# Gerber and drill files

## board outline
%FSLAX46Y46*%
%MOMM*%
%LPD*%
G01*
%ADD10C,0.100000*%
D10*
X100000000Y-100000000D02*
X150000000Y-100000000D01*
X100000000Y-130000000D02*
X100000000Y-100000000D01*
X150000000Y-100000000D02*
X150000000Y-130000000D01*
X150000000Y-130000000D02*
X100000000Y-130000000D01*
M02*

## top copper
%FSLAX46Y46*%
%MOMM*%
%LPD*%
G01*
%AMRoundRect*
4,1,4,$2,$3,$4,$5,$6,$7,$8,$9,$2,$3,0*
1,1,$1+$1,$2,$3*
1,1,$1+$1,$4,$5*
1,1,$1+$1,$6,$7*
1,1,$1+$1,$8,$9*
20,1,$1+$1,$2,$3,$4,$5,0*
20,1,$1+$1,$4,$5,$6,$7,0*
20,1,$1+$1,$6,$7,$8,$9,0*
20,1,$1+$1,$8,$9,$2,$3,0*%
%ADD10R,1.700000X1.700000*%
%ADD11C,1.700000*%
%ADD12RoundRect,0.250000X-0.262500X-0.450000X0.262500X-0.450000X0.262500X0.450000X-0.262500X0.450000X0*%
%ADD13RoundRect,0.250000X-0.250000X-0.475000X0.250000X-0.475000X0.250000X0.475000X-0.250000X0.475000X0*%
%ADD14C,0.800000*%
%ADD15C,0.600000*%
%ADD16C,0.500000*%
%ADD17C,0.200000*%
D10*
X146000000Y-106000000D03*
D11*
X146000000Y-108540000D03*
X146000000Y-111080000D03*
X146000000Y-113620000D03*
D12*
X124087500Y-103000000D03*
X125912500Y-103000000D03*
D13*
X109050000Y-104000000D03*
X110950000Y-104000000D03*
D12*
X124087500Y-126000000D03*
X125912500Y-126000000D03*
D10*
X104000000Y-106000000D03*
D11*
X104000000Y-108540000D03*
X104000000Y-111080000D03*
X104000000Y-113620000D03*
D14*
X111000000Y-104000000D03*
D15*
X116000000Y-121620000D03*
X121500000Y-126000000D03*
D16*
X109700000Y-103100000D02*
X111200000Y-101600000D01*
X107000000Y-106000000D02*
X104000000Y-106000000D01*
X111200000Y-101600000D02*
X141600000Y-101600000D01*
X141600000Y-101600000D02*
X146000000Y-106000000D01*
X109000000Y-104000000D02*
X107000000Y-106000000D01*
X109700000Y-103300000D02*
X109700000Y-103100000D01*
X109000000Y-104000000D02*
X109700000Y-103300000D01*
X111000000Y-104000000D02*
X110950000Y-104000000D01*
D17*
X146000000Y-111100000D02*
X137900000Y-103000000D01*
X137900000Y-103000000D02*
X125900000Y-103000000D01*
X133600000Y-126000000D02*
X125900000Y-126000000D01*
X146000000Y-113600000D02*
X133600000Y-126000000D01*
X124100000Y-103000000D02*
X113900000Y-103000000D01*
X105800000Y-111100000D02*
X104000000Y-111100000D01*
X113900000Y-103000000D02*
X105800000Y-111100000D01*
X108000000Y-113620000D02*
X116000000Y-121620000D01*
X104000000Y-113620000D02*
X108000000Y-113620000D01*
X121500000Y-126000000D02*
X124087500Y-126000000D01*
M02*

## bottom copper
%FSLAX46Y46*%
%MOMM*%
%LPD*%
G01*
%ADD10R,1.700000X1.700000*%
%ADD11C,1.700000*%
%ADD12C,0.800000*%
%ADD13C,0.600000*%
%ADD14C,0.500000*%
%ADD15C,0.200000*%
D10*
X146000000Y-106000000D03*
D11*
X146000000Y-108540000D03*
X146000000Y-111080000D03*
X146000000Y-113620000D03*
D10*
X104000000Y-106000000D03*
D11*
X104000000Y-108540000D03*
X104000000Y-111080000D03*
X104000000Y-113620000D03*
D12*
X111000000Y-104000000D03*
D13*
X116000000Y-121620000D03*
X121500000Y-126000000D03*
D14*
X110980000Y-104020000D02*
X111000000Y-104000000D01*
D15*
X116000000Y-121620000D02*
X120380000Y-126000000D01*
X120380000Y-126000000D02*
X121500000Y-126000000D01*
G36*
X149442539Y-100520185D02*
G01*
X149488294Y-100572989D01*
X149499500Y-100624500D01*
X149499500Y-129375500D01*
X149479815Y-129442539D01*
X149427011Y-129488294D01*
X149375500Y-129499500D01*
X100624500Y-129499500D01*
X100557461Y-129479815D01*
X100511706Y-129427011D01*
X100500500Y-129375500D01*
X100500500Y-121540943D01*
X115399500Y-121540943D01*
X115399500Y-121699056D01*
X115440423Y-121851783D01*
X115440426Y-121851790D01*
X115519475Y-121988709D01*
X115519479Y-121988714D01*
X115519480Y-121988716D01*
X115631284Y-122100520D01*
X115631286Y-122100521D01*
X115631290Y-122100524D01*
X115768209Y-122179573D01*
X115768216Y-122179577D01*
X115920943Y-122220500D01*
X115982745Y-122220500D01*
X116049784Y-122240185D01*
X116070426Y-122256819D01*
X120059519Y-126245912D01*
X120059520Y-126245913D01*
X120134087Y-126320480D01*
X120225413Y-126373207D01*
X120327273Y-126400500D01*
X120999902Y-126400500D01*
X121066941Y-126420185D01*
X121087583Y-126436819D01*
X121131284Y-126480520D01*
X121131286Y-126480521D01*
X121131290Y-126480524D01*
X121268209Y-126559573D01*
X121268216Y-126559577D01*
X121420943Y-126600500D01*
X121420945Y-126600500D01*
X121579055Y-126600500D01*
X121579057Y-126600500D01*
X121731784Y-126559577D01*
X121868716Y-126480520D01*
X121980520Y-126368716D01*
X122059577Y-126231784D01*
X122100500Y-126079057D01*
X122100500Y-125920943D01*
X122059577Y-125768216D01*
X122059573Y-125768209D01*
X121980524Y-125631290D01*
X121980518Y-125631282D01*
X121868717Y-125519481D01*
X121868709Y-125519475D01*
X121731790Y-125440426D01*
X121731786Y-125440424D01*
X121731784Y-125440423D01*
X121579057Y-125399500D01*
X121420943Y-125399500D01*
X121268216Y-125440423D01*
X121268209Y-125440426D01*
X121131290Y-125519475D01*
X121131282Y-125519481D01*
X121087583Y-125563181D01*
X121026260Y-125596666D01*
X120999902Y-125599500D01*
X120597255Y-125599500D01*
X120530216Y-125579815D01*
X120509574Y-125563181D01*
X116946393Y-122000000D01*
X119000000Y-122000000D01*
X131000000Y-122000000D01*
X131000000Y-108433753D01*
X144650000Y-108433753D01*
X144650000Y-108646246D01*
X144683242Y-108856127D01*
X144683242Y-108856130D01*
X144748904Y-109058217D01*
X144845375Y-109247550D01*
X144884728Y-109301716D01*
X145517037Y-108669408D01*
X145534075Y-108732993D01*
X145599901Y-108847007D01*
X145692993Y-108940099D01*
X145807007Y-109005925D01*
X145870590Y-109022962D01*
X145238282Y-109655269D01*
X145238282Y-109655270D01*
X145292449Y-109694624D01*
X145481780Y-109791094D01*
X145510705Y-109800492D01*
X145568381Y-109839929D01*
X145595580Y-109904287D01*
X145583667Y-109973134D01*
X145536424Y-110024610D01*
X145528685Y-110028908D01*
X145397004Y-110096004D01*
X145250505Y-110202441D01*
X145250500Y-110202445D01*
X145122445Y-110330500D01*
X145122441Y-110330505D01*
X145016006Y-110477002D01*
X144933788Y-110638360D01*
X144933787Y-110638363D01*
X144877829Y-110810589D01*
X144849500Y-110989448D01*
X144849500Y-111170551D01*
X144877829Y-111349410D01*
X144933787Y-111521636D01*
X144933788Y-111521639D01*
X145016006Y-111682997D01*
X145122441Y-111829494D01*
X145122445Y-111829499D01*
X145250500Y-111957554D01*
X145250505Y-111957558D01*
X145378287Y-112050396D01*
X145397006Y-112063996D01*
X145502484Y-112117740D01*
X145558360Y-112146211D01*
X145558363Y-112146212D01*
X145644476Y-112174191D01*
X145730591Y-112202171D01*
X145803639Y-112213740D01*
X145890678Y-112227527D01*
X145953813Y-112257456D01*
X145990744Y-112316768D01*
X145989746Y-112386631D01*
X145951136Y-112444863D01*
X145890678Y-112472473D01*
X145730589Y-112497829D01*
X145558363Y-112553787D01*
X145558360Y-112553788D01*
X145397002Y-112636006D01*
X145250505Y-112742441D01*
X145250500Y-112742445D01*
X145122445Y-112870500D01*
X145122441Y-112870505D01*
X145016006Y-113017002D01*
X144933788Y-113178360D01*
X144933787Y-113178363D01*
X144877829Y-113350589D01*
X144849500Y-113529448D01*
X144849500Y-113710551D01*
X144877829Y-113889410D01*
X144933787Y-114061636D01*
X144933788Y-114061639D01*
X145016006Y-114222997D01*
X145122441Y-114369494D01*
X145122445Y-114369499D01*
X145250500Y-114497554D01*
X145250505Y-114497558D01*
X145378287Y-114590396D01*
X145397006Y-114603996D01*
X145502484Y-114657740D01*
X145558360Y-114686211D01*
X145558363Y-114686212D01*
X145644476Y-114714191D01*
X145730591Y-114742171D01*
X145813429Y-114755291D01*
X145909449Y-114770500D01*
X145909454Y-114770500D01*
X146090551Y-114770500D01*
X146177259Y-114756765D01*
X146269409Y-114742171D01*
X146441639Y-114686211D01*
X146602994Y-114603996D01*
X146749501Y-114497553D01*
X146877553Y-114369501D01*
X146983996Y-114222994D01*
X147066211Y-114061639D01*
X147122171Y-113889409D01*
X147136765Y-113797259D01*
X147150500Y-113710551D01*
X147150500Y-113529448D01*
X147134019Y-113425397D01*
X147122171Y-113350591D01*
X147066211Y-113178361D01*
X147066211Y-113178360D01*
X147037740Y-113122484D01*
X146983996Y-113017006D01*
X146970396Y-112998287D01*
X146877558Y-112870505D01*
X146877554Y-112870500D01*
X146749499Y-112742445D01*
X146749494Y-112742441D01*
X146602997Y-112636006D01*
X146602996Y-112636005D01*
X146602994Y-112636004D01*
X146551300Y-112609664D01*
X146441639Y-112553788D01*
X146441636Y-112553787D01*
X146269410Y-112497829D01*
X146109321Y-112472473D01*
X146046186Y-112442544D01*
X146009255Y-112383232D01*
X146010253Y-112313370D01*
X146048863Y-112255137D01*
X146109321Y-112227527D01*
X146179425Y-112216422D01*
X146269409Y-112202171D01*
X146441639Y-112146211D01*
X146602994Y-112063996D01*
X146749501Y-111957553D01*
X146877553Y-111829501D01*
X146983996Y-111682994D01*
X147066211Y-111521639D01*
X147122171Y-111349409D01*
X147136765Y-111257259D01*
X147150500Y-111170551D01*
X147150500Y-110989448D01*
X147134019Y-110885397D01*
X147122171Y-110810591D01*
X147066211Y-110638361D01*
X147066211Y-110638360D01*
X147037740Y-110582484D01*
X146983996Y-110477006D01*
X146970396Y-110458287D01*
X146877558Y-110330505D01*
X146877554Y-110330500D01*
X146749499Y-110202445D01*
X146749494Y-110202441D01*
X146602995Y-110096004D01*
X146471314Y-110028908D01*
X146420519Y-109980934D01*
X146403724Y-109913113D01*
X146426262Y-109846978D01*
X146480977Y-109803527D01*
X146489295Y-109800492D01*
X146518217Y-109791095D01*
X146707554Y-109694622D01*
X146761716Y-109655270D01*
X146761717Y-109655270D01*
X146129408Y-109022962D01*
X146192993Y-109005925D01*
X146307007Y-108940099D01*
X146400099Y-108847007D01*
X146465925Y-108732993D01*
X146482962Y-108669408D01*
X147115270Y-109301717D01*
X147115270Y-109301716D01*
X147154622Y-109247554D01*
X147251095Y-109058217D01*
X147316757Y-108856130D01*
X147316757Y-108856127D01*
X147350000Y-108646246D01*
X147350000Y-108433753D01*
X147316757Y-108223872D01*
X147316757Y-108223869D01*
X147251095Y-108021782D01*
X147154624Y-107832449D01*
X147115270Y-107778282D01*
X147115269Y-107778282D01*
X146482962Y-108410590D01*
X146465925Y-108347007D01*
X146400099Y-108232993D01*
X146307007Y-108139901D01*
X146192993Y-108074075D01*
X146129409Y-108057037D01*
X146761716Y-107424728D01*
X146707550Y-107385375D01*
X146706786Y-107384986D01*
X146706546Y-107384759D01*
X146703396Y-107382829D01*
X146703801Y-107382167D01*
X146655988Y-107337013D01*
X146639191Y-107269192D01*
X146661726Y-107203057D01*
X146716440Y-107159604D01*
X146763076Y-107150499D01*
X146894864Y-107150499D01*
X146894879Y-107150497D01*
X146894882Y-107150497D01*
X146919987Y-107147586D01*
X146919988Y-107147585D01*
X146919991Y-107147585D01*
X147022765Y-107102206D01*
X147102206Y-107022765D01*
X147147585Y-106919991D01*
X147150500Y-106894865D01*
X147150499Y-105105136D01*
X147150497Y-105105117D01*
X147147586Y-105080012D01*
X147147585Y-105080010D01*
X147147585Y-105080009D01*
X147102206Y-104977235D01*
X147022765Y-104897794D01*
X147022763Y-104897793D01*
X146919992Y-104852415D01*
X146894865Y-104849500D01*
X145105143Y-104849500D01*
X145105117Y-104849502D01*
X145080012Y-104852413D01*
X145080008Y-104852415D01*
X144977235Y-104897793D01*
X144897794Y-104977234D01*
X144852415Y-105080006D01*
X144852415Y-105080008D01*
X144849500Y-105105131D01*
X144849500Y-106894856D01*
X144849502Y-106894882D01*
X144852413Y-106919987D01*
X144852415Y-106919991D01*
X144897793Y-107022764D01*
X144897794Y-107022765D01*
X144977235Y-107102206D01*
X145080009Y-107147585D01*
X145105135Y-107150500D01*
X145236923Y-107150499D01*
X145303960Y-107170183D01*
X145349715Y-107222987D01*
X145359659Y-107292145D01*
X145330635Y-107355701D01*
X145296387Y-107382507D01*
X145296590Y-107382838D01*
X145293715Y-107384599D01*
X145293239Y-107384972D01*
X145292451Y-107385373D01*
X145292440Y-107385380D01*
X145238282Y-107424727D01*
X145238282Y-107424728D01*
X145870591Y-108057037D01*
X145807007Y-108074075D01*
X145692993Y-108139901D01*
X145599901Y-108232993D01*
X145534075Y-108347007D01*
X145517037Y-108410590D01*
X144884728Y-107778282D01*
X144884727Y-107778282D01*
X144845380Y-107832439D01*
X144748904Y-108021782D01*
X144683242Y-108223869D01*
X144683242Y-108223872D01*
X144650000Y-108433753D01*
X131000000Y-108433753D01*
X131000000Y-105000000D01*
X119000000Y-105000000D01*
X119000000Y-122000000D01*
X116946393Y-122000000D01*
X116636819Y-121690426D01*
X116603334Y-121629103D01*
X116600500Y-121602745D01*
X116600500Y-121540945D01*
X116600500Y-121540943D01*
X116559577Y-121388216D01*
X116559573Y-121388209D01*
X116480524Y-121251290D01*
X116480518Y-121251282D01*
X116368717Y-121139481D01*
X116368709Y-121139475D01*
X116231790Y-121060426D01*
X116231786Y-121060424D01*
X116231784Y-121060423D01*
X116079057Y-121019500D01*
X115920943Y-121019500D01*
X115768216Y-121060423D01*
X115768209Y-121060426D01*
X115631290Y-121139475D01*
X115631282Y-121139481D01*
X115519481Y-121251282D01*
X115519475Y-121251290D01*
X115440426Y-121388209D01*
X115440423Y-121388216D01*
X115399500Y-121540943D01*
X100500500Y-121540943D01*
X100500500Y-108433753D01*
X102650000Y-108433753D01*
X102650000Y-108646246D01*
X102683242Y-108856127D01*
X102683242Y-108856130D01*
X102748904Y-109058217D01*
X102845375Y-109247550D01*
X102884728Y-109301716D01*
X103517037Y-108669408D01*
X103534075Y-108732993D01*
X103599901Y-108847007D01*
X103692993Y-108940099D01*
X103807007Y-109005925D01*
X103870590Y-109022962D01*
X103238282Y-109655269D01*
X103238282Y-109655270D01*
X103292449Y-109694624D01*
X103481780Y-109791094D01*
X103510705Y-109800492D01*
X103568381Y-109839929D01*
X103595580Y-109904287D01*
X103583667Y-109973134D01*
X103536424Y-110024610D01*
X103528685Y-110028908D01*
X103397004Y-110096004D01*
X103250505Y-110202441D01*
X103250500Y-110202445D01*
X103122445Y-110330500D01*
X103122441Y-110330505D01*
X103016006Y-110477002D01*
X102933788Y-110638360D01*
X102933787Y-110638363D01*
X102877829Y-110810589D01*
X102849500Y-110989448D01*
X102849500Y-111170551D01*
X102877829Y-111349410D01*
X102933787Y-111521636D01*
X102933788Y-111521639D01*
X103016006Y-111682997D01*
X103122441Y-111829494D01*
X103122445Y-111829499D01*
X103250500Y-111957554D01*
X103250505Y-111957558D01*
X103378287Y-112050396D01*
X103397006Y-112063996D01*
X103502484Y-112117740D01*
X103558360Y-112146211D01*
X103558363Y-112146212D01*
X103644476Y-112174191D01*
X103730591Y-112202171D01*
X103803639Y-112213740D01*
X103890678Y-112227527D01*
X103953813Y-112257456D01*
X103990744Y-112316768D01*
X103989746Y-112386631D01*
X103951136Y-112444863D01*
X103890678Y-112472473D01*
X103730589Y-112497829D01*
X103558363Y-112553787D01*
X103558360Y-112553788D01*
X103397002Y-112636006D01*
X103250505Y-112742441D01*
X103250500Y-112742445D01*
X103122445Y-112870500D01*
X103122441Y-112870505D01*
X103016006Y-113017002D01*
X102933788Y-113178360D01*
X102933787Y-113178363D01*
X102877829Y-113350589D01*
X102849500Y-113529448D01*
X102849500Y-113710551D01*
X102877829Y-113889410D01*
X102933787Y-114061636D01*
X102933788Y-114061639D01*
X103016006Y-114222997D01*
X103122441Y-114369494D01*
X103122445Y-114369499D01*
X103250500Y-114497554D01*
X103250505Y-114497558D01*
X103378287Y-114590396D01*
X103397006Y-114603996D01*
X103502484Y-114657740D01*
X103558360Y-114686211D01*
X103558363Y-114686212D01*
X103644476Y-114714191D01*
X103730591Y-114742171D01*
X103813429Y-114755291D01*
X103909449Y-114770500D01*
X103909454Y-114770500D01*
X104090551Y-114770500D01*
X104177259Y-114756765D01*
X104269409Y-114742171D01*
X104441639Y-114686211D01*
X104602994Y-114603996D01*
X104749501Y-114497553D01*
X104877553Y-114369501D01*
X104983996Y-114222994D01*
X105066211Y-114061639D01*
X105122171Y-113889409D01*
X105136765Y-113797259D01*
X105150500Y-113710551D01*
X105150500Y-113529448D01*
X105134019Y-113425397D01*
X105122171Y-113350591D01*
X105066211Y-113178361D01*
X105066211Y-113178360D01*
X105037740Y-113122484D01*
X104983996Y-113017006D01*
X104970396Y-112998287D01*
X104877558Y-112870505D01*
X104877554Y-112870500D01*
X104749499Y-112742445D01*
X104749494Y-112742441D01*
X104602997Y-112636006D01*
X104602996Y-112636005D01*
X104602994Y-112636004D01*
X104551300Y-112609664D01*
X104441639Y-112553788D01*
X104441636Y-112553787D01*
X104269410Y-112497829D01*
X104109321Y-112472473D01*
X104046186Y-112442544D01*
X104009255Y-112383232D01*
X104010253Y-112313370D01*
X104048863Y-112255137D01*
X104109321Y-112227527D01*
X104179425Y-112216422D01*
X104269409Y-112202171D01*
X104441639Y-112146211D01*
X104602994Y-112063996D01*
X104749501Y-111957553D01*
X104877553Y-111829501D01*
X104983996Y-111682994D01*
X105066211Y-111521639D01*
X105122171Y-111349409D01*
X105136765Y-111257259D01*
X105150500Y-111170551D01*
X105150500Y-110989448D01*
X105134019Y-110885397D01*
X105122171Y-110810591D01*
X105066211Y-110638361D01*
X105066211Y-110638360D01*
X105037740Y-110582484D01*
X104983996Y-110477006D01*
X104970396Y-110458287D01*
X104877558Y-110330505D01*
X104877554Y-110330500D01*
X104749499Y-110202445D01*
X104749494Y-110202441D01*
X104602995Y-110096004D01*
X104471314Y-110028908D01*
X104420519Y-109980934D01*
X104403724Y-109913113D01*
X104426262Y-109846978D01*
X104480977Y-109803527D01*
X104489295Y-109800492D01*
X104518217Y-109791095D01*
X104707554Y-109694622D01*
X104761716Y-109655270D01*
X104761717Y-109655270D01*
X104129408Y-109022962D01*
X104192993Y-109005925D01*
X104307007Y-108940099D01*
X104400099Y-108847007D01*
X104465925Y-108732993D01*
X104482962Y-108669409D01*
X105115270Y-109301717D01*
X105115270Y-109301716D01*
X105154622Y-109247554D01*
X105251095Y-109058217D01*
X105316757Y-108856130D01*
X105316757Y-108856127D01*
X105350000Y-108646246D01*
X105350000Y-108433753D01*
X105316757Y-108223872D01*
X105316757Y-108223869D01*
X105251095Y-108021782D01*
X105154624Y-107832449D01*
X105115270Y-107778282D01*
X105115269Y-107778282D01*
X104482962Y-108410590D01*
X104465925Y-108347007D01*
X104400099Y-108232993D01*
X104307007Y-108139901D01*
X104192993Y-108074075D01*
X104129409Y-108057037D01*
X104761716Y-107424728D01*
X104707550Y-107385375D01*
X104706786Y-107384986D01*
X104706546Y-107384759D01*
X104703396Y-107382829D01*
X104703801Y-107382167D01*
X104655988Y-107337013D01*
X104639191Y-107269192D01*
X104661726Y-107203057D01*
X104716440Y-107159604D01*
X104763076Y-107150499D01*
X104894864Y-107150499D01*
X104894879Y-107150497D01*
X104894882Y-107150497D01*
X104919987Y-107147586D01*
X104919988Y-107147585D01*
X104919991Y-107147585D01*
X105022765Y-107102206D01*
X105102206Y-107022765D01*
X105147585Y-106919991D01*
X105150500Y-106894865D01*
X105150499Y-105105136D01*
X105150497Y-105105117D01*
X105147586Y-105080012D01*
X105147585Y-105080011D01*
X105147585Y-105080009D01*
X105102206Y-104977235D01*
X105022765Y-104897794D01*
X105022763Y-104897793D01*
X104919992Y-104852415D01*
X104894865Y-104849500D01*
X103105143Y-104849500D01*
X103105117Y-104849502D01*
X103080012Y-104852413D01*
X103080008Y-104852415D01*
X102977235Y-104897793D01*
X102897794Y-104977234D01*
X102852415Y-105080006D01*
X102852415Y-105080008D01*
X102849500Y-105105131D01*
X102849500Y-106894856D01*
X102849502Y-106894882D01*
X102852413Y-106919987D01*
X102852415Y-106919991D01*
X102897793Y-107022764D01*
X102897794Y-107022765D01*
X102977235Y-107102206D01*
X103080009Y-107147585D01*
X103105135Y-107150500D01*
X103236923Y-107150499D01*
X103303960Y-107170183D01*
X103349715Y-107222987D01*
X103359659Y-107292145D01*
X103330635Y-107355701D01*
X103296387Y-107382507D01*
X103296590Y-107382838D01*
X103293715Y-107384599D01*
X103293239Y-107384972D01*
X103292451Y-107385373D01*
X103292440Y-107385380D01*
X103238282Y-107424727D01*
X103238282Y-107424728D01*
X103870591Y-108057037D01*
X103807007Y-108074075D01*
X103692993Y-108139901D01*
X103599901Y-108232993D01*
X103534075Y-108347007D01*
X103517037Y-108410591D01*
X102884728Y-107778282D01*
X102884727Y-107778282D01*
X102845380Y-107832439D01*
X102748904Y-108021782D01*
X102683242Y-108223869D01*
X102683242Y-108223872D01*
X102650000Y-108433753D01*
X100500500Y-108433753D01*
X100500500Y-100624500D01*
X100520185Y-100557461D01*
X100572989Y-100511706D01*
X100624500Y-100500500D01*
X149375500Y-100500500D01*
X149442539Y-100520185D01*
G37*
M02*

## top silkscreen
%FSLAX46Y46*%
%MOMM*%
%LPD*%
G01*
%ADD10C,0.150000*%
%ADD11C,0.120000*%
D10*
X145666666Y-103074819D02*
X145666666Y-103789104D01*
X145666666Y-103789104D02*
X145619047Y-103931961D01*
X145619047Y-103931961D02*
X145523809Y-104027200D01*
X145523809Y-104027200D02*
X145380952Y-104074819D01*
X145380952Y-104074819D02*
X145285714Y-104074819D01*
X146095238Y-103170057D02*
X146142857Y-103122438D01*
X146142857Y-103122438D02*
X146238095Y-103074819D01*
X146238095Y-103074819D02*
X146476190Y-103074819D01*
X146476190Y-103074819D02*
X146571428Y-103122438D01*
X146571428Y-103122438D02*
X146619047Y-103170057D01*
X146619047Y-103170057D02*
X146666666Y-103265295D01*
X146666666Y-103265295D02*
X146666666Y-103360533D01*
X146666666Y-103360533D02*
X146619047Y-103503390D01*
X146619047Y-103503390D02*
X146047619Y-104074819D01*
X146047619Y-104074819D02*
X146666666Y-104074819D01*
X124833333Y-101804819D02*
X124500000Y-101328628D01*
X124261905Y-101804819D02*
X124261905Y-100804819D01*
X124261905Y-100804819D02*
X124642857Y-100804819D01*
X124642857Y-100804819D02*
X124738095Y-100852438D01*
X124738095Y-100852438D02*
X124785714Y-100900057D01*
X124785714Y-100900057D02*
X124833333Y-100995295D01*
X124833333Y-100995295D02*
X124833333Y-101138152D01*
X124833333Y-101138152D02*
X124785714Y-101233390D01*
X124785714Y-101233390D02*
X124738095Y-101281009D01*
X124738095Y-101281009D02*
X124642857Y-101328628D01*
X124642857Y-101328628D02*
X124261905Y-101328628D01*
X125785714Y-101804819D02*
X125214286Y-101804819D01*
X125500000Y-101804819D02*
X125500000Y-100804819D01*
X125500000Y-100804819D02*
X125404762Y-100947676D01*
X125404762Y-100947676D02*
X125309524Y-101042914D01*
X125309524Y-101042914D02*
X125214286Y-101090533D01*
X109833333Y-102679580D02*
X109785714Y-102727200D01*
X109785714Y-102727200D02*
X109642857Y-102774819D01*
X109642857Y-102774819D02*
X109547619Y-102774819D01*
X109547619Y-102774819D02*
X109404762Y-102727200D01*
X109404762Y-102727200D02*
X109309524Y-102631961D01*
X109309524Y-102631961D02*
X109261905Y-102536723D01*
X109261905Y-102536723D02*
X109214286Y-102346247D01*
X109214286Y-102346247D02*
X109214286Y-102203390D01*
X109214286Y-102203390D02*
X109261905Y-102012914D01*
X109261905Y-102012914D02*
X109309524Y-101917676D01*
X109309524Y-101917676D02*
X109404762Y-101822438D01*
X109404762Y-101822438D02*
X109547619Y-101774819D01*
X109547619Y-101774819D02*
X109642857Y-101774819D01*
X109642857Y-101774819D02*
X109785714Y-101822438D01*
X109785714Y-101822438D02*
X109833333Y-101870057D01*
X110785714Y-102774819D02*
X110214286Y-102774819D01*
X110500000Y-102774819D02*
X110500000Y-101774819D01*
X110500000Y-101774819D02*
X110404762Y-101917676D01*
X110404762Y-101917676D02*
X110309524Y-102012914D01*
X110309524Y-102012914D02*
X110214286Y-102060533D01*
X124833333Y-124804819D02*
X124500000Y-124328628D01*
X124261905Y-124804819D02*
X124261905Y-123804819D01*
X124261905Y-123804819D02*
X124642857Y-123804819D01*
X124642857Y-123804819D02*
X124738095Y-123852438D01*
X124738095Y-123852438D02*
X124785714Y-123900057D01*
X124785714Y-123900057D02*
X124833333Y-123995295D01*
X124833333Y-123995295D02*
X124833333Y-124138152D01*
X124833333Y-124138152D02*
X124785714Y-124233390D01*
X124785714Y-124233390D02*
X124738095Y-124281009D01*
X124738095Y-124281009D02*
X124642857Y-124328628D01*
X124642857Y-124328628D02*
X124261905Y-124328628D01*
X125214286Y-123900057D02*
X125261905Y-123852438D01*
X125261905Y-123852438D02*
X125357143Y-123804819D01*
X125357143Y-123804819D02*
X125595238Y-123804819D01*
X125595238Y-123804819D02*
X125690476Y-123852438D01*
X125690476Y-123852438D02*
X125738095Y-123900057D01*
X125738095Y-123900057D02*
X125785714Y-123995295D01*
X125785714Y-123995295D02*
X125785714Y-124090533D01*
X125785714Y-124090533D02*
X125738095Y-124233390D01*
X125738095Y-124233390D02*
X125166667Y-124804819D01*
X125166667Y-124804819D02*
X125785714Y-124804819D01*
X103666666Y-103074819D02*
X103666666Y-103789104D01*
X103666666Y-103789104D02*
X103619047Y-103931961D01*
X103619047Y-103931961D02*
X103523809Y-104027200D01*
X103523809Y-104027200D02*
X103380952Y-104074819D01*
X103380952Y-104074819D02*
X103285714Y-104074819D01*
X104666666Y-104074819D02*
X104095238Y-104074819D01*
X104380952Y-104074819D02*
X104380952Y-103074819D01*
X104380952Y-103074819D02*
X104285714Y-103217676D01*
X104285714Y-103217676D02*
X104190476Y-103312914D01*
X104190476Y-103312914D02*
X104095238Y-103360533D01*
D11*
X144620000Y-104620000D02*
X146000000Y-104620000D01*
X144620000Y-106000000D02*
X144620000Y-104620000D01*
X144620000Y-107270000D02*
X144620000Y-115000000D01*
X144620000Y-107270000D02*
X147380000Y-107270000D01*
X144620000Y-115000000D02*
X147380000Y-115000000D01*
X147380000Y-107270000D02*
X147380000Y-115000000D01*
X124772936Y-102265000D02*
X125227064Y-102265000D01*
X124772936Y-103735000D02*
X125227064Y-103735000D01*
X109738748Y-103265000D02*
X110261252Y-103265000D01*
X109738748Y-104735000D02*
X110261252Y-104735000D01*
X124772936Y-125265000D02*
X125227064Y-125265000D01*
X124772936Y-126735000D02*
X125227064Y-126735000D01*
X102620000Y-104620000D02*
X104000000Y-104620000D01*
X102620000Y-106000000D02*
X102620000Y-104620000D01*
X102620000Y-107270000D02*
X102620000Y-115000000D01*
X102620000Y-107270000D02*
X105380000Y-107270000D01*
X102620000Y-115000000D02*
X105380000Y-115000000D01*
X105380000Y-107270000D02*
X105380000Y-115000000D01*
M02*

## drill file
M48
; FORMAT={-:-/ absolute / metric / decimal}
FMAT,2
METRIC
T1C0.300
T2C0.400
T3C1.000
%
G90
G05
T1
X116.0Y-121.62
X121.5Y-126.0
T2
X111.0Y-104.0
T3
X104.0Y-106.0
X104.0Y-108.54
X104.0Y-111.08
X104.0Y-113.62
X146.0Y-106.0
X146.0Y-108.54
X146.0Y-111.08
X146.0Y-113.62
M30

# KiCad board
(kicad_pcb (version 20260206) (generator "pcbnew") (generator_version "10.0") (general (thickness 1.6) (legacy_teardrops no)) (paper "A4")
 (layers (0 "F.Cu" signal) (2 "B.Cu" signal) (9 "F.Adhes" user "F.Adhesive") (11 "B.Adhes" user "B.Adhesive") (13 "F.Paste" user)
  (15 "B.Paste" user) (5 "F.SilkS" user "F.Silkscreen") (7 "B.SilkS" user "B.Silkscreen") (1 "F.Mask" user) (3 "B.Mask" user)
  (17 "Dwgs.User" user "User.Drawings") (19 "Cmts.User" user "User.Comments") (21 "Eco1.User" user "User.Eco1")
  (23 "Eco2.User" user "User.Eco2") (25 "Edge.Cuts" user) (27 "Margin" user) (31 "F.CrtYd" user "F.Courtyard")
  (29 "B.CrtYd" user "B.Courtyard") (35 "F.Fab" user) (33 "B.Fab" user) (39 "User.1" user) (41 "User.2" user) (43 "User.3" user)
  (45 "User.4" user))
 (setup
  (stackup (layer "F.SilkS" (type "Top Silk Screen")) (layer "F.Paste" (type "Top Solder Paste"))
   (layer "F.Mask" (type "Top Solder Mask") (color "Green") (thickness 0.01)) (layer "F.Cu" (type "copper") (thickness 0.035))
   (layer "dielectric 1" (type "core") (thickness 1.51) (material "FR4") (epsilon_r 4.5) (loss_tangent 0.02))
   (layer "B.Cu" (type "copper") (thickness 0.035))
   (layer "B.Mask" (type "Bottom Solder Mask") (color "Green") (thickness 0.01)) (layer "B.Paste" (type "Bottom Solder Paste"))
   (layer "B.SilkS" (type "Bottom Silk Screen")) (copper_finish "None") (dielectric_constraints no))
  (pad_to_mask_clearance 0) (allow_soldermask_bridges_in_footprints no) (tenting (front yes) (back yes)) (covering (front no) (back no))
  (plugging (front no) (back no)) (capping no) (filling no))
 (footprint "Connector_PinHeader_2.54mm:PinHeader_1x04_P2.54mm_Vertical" (layer "F.Cu") (at 146 106)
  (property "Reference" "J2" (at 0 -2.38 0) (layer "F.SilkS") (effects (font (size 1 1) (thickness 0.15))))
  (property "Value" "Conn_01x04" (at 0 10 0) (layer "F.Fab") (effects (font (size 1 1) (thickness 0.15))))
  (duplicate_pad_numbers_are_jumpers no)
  (fp_line (start -1.38 -1.38) (end 0 -1.38) (stroke (width 0.12) (type solid)) (layer "F.SilkS"))
  (fp_line (start -1.38 0) (end -1.38 -1.38) (stroke (width 0.12) (type solid)) (layer "F.SilkS"))
  (fp_line (start -1.38 1.27) (end -1.38 9) (stroke (width 0.12) (type solid)) (layer "F.SilkS"))
  (fp_line (start -1.38 1.27) (end 1.38 1.27) (stroke (width 0.12) (type solid)) (layer "F.SilkS"))
  (fp_line (start -1.38 9) (end 1.38 9) (stroke (width 0.12) (type solid)) (layer "F.SilkS"))
  (fp_line (start 1.38 1.27) (end 1.38 9) (stroke (width 0.12) (type solid)) (layer "F.SilkS"))
  (pad "1" thru_hole rect (at 0 0) (size 1.7 1.7) (drill 1) (layers "*.Cu" "*.Mask") (remove_unused_layers no) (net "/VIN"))
  (pad "2" thru_hole circle (at 0 2.54) (size 1.7 1.7) (drill 1) (layers "*.Cu" "*.Mask") (remove_unused_layers no) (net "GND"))
  (pad "3" thru_hole circle (at 0 5.08) (size 1.7 1.7) (drill 1) (layers "*.Cu" "*.Mask") (remove_unused_layers no) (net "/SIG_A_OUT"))
  (pad "4" thru_hole circle (at 0 7.62) (size 1.7 1.7) (drill 1) (layers "*.Cu" "*.Mask") (remove_unused_layers no) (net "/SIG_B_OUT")))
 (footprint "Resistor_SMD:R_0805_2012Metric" (layer "F.Cu") (at 125 103)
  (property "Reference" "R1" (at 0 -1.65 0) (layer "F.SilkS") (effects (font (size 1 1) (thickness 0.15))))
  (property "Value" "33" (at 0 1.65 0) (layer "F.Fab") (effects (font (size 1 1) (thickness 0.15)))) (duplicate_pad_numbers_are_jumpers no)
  (fp_line (start -0.227064 -0.735) (end 0.227064 -0.735) (stroke (width 0.12) (type solid)) (layer "F.SilkS"))
  (fp_line (start -0.227064 0.735) (end 0.227064 0.735) (stroke (width 0.12) (type solid)) (layer "F.SilkS"))
  (pad "1" smd roundrect (at -0.9125 0) (size 1.025 1.4) (layers "F.Cu" "F.Mask" "F.Paste") (roundrect_rratio 0.243902) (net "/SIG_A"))
  (pad "2" smd roundrect (at 0.9125 0) (size 1.025 1.4) (layers "F.Cu" "F.Mask" "F.Paste") (roundrect_rratio 0.243902) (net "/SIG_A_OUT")))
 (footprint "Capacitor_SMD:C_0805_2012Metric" (layer "F.Cu") (at 110 104)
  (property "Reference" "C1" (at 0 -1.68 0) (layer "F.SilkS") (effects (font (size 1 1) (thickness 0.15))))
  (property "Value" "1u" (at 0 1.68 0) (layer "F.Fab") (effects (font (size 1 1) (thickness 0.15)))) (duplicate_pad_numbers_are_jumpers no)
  (fp_line (start -0.261252 -0.735) (end 0.261252 -0.735) (stroke (width 0.12) (type solid)) (layer "F.SilkS"))
  (fp_line (start -0.261252 0.735) (end 0.261252 0.735) (stroke (width 0.12) (type solid)) (layer "F.SilkS"))
  (pad "1" smd roundrect (at -0.95 0) (size 1 1.45) (layers "F.Cu" "F.Mask" "F.Paste") (roundrect_rratio 0.25) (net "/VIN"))
  (pad "2" smd roundrect (at 0.95 0) (size 1 1.45) (layers "F.Cu" "F.Mask" "F.Paste") (roundrect_rratio 0.25) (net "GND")))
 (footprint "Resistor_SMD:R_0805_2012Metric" (layer "F.Cu") (at 125 126)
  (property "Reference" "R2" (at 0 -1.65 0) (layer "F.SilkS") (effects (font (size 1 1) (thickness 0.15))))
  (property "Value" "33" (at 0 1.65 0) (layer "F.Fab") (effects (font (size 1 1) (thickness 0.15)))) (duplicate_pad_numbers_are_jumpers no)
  (fp_line (start -0.227064 -0.735) (end 0.227064 -0.735) (stroke (width 0.12) (type solid)) (layer "F.SilkS"))
  (fp_line (start -0.227064 0.735) (end 0.227064 0.735) (stroke (width 0.12) (type solid)) (layer "F.SilkS"))
  (pad "1" smd roundrect (at -0.9125 0) (size 1.025 1.4) (layers "F.Cu" "F.Mask" "F.Paste") (roundrect_rratio 0.243902) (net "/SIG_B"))
  (pad "2" smd roundrect (at 0.9125 0) (size 1.025 1.4) (layers "F.Cu" "F.Mask" "F.Paste") (roundrect_rratio 0.243902) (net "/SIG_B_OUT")))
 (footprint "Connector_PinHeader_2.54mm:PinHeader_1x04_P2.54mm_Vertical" (layer "F.Cu") (at 104 106)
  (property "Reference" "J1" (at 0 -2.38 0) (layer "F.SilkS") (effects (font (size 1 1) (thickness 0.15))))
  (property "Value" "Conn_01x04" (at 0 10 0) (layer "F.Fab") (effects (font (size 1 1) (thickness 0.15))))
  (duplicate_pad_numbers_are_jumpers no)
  (fp_line (start -1.38 -1.38) (end 0 -1.38) (stroke (width 0.12) (type solid)) (layer "F.SilkS"))
  (fp_line (start -1.38 0) (end -1.38 -1.38) (stroke (width 0.12) (type solid)) (layer "F.SilkS"))
  (fp_line (start -1.38 1.27) (end -1.38 9) (stroke (width 0.12) (type solid)) (layer "F.SilkS"))
  (fp_line (start -1.38 1.27) (end 1.38 1.27) (stroke (width 0.12) (type solid)) (layer "F.SilkS"))
  (fp_line (start -1.38 9) (end 1.38 9) (stroke (width 0.12) (type solid)) (layer "F.SilkS"))
  (fp_line (start 1.38 1.27) (end 1.38 9) (stroke (width 0.12) (type solid)) (layer "F.SilkS"))
  (pad "1" thru_hole rect (at 0 0) (size 1.7 1.7) (drill 1) (layers "*.Cu" "*.Mask") (remove_unused_layers no) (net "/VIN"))
  (pad "2" thru_hole circle (at 0 2.54) (size 1.7 1.7) (drill 1) (layers "*.Cu" "*.Mask") (remove_unused_layers no) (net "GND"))
  (pad "3" thru_hole circle (at 0 5.08) (size 1.7 1.7) (drill 1) (layers "*.Cu" "*.Mask") (remove_unused_layers no) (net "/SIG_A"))
  (pad "4" thru_hole circle (at 0 7.62) (size 1.7 1.7) (drill 1) (layers "*.Cu" "*.Mask") (remove_unused_layers no) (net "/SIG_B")))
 (gr_line (start 100 100) (end 150 100) (stroke (width 0.1) (type default)) (layer "Edge.Cuts"))
 (gr_line (start 100 130) (end 100 100) (stroke (width 0.1) (type default)) (layer "Edge.Cuts"))
 (gr_line (start 150 100) (end 150 130) (stroke (width 0.1) (type default)) (layer "Edge.Cuts"))
 (gr_line (start 150 130) (end 100 130) (stroke (width 0.1) (type default)) (layer "Edge.Cuts"))
 (segment (start 109.7 103.1) (end 111.2 101.6) (width 0.5) (layer "F.Cu") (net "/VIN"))
 (segment (start 107 106) (end 104 106) (width 0.5) (layer "F.Cu") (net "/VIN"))
 (segment (start 111.2 101.6) (end 141.6 101.6) (width 0.5) (layer "F.Cu") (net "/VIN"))
 (segment (start 141.6 101.6) (end 146 106) (width 0.5) (layer "F.Cu") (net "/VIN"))
 (segment (start 109 104) (end 107 106) (width 0.5) (layer "F.Cu") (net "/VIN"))
 (segment (start 109.7 103.3) (end 109.7 103.1) (width 0.5) (layer "F.Cu") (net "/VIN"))
 (segment (start 109 104) (end 109.7 103.3) (width 0.5) (layer "F.Cu") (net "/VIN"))
 (segment (start 111 104) (end 110.95 104) (width 0.5) (layer "F.Cu") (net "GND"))
 (via (at 111 104) (size 0.8) (drill 0.4) (layers "F.Cu" "B.Cu") (capping yes) (filling yes) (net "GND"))
 (segment (start 110.98 104.02) (end 111 104) (width 0.5) (layer "B.Cu") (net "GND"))
 (segment (start 146 111.1) (end 137.9 103) (width 0.2) (layer "F.Cu") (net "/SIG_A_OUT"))
 (segment (start 137.9 103) (end 125.9 103) (width 0.2) (layer "F.Cu") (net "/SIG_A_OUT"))
 (segment (start 133.6 126) (end 125.9 126) (width 0.2) (layer "F.Cu") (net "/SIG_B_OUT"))
 (segment (start 146 113.6) (end 133.6 126) (width 0.2) (layer "F.Cu") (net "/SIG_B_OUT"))
 (segment (start 124.1 103) (end 113.9 103) (width 0.2) (layer "F.Cu") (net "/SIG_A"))
 (segment (start 105.8 111.1) (end 104 111.1) (width 0.2) (layer "F.Cu") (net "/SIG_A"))
 (segment (start 113.9 103) (end 105.8 111.1) (width 0.2) (layer "F.Cu") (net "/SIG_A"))
 (segment (start 108 113.62) (end 116 121.62) (width 0.2) (locked yes) (layer "F.Cu") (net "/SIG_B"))
 (segment (start 104 113.62) (end 108 113.62) (width 0.2) (locked yes) (layer "F.Cu") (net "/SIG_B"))
 (segment (start 121.5 126) (end 124.0875 126) (width 0.2) (locked yes) (layer "F.Cu") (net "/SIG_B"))
 (via (at 116 121.62) (size 0.6) (drill 0.3) (layers "F.Cu" "B.Cu") (locked yes) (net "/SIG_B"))
 (via (at 121.5 126) (size 0.6) (drill 0.3) (layers "F.Cu" "B.Cu") (locked yes) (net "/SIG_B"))
 (segment (start 116 121.62) (end 120.38 126) (width 0.2) (locked yes) (layer "B.Cu") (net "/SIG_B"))
 (segment (start 120.38 126) (end 121.5 126) (width 0.2) (locked yes) (layer "B.Cu") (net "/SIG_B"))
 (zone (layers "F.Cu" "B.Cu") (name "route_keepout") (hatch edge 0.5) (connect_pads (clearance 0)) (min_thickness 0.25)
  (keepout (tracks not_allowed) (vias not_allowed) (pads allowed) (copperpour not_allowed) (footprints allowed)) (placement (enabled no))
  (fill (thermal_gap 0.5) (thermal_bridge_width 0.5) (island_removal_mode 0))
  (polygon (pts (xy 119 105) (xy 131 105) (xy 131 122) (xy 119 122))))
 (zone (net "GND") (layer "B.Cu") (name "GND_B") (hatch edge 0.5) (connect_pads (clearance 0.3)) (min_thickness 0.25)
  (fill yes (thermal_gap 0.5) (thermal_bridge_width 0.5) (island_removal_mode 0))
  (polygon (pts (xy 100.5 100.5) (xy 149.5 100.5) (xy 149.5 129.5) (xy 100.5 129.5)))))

